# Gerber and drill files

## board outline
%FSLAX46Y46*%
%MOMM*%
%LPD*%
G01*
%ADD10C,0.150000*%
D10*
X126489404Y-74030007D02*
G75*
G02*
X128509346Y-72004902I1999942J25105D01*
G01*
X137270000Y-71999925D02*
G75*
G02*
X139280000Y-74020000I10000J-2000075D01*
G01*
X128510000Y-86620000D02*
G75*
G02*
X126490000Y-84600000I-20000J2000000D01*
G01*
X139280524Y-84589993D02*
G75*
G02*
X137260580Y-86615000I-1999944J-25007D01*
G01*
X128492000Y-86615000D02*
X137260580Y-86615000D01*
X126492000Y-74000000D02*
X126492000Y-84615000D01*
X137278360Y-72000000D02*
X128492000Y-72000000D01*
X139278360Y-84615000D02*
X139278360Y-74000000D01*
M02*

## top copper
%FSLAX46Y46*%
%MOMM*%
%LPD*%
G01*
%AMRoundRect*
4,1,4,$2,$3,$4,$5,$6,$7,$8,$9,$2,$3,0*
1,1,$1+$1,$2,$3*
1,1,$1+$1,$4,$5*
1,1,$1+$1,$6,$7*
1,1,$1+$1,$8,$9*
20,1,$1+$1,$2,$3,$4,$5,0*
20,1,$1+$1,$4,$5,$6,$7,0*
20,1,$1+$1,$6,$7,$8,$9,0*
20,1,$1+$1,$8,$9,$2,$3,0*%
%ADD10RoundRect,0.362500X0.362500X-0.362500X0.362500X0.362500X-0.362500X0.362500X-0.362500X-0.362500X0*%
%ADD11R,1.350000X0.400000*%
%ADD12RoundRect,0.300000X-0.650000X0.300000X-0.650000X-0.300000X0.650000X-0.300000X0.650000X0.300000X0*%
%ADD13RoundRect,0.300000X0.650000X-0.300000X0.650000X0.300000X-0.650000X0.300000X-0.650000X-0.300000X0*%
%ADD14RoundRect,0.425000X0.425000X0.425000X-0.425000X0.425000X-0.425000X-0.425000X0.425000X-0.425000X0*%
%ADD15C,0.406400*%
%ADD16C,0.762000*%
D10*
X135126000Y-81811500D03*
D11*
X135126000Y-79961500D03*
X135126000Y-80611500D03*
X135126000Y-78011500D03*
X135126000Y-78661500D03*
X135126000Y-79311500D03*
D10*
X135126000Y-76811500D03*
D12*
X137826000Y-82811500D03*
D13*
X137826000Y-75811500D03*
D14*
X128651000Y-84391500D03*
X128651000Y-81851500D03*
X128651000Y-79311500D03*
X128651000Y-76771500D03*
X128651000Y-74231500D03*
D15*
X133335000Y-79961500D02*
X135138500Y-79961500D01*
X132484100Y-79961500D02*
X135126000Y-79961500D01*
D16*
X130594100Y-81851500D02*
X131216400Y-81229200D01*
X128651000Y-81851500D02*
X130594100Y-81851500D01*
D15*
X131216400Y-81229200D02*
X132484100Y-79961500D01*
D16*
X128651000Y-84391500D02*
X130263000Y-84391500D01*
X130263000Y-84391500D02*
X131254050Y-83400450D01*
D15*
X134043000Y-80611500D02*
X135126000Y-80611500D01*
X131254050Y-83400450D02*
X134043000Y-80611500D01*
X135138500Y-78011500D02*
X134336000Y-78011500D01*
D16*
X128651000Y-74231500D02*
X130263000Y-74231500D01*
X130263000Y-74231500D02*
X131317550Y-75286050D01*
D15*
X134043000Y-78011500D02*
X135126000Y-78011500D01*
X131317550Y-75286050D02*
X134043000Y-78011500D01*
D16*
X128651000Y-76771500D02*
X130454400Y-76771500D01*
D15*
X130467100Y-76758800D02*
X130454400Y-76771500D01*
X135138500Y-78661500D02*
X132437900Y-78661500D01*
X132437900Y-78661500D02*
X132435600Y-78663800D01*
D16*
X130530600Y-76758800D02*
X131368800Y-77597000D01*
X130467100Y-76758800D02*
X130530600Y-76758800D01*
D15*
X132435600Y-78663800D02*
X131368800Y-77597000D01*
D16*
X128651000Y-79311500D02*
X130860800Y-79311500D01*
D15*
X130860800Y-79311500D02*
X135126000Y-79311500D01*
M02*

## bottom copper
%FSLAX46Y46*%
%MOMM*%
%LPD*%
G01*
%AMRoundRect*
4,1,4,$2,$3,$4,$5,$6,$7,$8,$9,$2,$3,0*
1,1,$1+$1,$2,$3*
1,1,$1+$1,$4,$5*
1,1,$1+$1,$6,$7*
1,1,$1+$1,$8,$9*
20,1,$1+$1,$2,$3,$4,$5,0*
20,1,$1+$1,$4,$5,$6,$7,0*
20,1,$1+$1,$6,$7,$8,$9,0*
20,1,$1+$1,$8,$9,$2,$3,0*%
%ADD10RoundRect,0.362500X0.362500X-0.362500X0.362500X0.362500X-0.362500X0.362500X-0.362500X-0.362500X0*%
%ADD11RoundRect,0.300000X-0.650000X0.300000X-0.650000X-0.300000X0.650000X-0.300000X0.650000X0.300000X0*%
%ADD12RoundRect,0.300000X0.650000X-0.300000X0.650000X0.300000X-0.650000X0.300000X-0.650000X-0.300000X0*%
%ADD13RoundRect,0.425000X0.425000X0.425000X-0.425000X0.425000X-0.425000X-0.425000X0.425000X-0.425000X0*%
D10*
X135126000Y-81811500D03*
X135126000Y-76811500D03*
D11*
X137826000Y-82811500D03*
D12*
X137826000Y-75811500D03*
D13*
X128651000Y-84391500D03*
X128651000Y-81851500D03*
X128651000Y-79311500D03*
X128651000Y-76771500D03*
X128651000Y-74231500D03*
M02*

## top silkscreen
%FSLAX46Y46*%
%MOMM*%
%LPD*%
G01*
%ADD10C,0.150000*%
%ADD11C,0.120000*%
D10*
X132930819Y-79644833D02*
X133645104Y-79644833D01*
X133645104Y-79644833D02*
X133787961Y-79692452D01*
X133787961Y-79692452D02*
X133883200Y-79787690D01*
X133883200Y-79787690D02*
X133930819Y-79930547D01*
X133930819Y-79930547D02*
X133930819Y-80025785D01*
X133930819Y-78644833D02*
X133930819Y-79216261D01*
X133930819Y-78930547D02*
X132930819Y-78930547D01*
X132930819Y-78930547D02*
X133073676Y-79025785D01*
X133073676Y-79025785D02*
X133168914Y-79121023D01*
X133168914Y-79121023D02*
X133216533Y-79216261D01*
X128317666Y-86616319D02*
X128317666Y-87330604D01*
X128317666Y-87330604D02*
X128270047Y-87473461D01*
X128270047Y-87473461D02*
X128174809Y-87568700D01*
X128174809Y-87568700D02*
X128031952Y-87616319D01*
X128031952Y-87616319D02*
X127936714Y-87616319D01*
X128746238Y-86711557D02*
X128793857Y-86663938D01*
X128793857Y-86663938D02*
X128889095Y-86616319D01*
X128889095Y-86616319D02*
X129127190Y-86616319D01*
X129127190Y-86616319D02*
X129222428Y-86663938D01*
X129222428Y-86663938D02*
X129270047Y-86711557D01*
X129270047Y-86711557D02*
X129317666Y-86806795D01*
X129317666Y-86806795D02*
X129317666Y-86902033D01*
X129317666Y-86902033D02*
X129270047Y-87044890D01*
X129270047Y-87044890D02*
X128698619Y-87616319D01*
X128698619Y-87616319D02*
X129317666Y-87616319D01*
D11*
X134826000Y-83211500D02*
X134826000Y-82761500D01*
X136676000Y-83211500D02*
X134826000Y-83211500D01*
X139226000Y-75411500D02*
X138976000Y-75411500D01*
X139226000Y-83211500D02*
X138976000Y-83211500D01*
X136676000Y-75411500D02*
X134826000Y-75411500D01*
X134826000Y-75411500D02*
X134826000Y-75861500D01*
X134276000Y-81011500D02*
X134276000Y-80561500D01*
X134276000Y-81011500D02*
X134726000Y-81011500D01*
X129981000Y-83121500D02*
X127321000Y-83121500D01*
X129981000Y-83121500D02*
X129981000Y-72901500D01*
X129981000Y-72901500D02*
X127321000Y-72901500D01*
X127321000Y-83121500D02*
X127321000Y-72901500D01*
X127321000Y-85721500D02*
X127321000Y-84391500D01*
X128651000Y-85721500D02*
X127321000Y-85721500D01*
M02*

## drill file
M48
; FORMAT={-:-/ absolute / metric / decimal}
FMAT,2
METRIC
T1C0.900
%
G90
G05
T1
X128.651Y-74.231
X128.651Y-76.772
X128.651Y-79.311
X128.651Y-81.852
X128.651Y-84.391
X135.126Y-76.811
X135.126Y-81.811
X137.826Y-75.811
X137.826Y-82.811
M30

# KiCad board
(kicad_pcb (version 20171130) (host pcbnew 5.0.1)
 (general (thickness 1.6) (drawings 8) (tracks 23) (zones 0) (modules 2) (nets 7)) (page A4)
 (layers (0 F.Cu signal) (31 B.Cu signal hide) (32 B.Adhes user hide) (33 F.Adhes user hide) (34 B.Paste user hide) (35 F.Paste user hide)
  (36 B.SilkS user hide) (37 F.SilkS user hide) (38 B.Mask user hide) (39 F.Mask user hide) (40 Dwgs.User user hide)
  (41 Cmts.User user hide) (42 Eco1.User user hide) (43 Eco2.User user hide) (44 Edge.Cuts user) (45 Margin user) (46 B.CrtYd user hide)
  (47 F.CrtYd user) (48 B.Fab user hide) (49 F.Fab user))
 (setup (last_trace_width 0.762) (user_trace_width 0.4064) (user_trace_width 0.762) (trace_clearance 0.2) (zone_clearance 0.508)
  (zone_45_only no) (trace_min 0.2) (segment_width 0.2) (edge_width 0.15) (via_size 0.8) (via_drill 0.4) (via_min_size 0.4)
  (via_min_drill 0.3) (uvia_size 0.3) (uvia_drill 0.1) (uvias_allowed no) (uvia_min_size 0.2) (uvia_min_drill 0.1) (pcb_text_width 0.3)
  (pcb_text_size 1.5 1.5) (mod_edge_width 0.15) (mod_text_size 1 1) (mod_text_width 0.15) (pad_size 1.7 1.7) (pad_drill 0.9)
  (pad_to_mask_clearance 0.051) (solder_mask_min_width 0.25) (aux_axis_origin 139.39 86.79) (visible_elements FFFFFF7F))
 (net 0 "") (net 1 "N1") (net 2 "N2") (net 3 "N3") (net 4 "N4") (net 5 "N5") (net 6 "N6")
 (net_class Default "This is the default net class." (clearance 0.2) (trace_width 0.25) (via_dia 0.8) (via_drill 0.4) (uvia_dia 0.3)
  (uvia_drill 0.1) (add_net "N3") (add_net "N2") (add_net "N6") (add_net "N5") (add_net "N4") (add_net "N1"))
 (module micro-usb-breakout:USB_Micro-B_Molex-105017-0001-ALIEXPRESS (layer F.Cu) (at 136.5885 79.3115 90)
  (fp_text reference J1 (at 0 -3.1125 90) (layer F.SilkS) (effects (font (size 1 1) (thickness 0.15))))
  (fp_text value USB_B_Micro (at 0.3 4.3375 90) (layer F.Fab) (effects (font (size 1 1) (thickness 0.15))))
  (fp_line (start -3.9 -1.7625) (end -3.45 -1.7625) (layer F.SilkS) (width 0.12))
  (fp_line (start -3.9 0.0875) (end -3.9 -1.7625) (layer F.SilkS) (width 0.12))
  (fp_line (start 3.9 2.6375) (end 3.9 2.3875) (layer F.SilkS) (width 0.12))
  (fp_line (start -3.9 2.6375) (end -3.9 2.3875) (layer F.SilkS) (width 0.12))
  (fp_line (start 3.9 0.0875) (end 3.9 -1.7625) (layer F.SilkS) (width 0.12))
  (fp_line (start 3.9 -1.7625) (end 3.45 -1.7625) (layer F.SilkS) (width 0.12))
  (fp_line (start -1.7 -2.3125) (end -1.25 -2.3125) (layer F.SilkS) (width 0.12))
  (fp_line (start -1.7 -2.3125) (end -1.7 -1.8625) (layer F.SilkS) (width 0.12))
  (pad 6 smd rect (at 1 1.2375 90) (size 1.5 1.9) (layers F.Paste F.Mask) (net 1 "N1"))
  (pad "" thru_hole roundrect (at -2.5 -1.4625 90) (size 1.45 1.45) (drill 0.9) (layers F.Cu F.Mask) (roundrect_rratio 0.25))
  (pad 2 smd rect (at -0.65 -1.4625 90) (size 0.4 1.35) (layers F.Cu F.Paste F.Mask) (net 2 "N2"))
  (pad 1 smd rect (at -1.3 -1.4625 90) (size 0.4 1.35) (layers F.Cu F.Paste F.Mask) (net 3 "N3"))
  (pad 5 smd rect (at 1.3 -1.4625 90) (size 0.4 1.35) (layers F.Cu F.Paste F.Mask) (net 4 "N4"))
  (pad 4 smd rect (at 0.65 -1.4625 90) (size 0.4 1.35) (layers F.Cu F.Paste F.Mask) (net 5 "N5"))
  (pad 3 smd rect (at 0 -1.4625 90) (size 0.4 1.35) (layers F.Cu F.Paste F.Mask) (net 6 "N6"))
  (pad "" thru_hole roundrect (at 2.5 -1.4625 90) (size 1.45 1.45) (drill 0.9) (layers F.Cu F.Mask) (roundrect_rratio 0.25))
  (pad 6 smd rect (at -1 1.2375 90) (size 1.5 1.9) (layers F.Paste F.Mask) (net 1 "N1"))
  (pad "" thru_hole roundrect (at -3.5 1.2375 270) (size 1.2 1.9) (drill 0.9) (layers F.Cu F.Mask) (roundrect_rratio 0.25))
  (pad "" thru_hole roundrect (at 3.5 1.2375 90) (size 1.2 1.9) (drill 0.9) (layers F.Cu F.Mask) (roundrect_rratio 0.25))
  (pad 6 smd rect (at 2.9 1.2375 90) (size 1.2 1.9) (layers F.Mask) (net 1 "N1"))
  (pad 6 smd rect (at -2.9 1.2375 90) (size 1.2 1.9) (layers F.Mask) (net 1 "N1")))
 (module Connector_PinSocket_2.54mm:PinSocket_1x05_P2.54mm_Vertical (layer F.Cu) (at 128.651 84.3915 180)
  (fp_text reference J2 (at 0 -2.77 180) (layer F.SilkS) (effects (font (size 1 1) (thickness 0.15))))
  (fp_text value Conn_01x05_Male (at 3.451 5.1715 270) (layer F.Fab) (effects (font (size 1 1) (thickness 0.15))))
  (fp_line (start -1.33 1.27) (end 1.33 1.27) (layer F.SilkS) (width 0.12))
  (fp_line (start -1.33 1.27) (end -1.33 11.49) (layer F.SilkS) (width 0.12))
  (fp_line (start -1.33 11.49) (end 1.33 11.49) (layer F.SilkS) (width 0.12))
  (fp_line (start 1.33 1.27) (end 1.33 11.49) (layer F.SilkS) (width 0.12))
  (fp_line (start 1.33 -1.33) (end 1.33 0) (layer F.SilkS) (width 0.12))
  (fp_line (start 0 -1.33) (end 1.33 -1.33) (layer F.SilkS) (width 0.12))
  (pad 1 thru_hole roundrect (at 0 0 180) (size 1.7 1.7) (drill 0.9) (layers F.Cu F.Mask) (roundrect_rratio 0.25) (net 3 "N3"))
  (pad 2 thru_hole roundrect (at 0 2.54 180) (size 1.7 1.7) (drill 0.9) (layers F.Cu F.Mask) (roundrect_rratio 0.25) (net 2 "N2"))
  (pad 3 thru_hole roundrect (at 0 5.08 180) (size 1.7 1.7) (drill 0.9) (layers F.Cu F.Mask) (roundrect_rratio 0.25) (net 6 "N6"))
  (pad 4 thru_hole roundrect (at 0 7.62 180) (size 1.7 1.7) (drill 0.9) (layers F.Cu F.Mask) (roundrect_rratio 0.25) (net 5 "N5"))
  (pad 5 thru_hole roundrect (at 0 10.16 180) (size 1.7 1.7) (drill 0.9) (layers F.Cu F.Mask) (roundrect_rratio 0.25) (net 4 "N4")))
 (gr_arc (start 128.489346 74.004902) (end 128.509346 72.004902) (angle -91.29214085) (layer Edge.Cuts) (width 0.15))
 (gr_arc (start 137.28 74) (end 139.28 74.02) (angle -90.85941521) (layer Edge.Cuts) (width 0.15))
 (gr_arc (start 128.49 84.62) (end 128.51 86.62) (angle 91.1458774) (layer Edge.Cuts) (width 0.15))
 (gr_arc (start 137.28058 84.615) (end 137.26058 86.615) (angle -91.28930637) (layer Edge.Cuts) (width 0.15))
 (gr_line (start 128.492 86.615) (end 137.26058 86.615) (layer Edge.Cuts) (width 0.15))
 (gr_line (start 126.492 74) (end 126.492 84.615) (layer Edge.Cuts) (width 0.15))
 (gr_line (start 137.27836 72) (end 128.492 72) (layer Edge.Cuts) (width 0.15))
 (gr_line (start 139.27836 84.615) (end 139.27836 74) (layer Edge.Cuts) (width 0.15))
 (segment (start 133.335 79.9615) (end 135.1385 79.9615) (width 0.4064) (layer F.Cu) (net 2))
 (segment (start 132.4841 79.9615) (end 135.126 79.9615) (width 0.4064) (layer F.Cu) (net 2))
 (segment (start 130.5941 81.8515) (end 131.2164 81.2292) (width 0.762) (layer F.Cu) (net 2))
 (segment (start 128.651 81.8515) (end 130.5941 81.8515) (width 0.762) (layer F.Cu) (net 2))
 (segment (start 131.2164 81.2292) (end 132.4841 79.9615) (width 0.4064) (layer F.Cu) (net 2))
 (segment (start 128.651 84.3915) (end 130.263 84.3915) (width 0.762) (layer F.Cu) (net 3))
 (segment (start 130.263 84.3915) (end 131.25405 83.40045) (width 0.762) (layer F.Cu) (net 3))
 (segment (start 134.043 80.6115) (end 135.126 80.6115) (width 0.4064) (layer F.Cu) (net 3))
 (segment (start 131.25405 83.40045) (end 134.043 80.6115) (width 0.4064) (layer F.Cu) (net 3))
 (segment (start 135.1385 78.0115) (end 134.336 78.0115) (width 0.4064) (layer F.Cu) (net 4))
 (segment (start 128.651 74.2315) (end 130.263 74.2315) (width 0.762) (layer F.Cu) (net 4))
 (segment (start 130.263 74.2315) (end 131.31755 75.28605) (width 0.762) (layer F.Cu) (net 4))
 (segment (start 134.043 78.0115) (end 135.126 78.0115) (width 0.4064) (layer F.Cu) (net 4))
 (segment (start 131.31755 75.28605) (end 134.043 78.0115) (width 0.4064) (layer F.Cu) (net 4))
 (segment (start 128.651 76.7715) (end 130.4544 76.7715) (width 0.762) (layer F.Cu) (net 5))
 (segment (start 130.4671 76.7588) (end 130.4544 76.7715) (width 0.4064) (layer F.Cu) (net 5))
 (segment (start 135.1385 78.6615) (end 132.4379 78.6615) (width 0.4064) (layer F.Cu) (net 5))
 (segment (start 132.4379 78.6615) (end 132.4356 78.6638) (width 0.4064) (layer F.Cu) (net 5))
 (segment (start 130.5306 76.7588) (end 131.3688 77.597) (width 0.762) (layer F.Cu) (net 5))
 (segment (start 130.4671 76.7588) (end 130.5306 76.7588) (width 0.762) (layer F.Cu) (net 5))
 (segment (start 132.4356 78.6638) (end 131.3688 77.597) (width 0.4064) (layer F.Cu) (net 5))
 (segment (start 128.651 79.3115) (end 130.8608 79.3115) (width 0.762) (layer F.Cu) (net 6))
 (segment (start 130.8608 79.3115) (end 135.126 79.3115) (width 0.4064) (layer F.Cu) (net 6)))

